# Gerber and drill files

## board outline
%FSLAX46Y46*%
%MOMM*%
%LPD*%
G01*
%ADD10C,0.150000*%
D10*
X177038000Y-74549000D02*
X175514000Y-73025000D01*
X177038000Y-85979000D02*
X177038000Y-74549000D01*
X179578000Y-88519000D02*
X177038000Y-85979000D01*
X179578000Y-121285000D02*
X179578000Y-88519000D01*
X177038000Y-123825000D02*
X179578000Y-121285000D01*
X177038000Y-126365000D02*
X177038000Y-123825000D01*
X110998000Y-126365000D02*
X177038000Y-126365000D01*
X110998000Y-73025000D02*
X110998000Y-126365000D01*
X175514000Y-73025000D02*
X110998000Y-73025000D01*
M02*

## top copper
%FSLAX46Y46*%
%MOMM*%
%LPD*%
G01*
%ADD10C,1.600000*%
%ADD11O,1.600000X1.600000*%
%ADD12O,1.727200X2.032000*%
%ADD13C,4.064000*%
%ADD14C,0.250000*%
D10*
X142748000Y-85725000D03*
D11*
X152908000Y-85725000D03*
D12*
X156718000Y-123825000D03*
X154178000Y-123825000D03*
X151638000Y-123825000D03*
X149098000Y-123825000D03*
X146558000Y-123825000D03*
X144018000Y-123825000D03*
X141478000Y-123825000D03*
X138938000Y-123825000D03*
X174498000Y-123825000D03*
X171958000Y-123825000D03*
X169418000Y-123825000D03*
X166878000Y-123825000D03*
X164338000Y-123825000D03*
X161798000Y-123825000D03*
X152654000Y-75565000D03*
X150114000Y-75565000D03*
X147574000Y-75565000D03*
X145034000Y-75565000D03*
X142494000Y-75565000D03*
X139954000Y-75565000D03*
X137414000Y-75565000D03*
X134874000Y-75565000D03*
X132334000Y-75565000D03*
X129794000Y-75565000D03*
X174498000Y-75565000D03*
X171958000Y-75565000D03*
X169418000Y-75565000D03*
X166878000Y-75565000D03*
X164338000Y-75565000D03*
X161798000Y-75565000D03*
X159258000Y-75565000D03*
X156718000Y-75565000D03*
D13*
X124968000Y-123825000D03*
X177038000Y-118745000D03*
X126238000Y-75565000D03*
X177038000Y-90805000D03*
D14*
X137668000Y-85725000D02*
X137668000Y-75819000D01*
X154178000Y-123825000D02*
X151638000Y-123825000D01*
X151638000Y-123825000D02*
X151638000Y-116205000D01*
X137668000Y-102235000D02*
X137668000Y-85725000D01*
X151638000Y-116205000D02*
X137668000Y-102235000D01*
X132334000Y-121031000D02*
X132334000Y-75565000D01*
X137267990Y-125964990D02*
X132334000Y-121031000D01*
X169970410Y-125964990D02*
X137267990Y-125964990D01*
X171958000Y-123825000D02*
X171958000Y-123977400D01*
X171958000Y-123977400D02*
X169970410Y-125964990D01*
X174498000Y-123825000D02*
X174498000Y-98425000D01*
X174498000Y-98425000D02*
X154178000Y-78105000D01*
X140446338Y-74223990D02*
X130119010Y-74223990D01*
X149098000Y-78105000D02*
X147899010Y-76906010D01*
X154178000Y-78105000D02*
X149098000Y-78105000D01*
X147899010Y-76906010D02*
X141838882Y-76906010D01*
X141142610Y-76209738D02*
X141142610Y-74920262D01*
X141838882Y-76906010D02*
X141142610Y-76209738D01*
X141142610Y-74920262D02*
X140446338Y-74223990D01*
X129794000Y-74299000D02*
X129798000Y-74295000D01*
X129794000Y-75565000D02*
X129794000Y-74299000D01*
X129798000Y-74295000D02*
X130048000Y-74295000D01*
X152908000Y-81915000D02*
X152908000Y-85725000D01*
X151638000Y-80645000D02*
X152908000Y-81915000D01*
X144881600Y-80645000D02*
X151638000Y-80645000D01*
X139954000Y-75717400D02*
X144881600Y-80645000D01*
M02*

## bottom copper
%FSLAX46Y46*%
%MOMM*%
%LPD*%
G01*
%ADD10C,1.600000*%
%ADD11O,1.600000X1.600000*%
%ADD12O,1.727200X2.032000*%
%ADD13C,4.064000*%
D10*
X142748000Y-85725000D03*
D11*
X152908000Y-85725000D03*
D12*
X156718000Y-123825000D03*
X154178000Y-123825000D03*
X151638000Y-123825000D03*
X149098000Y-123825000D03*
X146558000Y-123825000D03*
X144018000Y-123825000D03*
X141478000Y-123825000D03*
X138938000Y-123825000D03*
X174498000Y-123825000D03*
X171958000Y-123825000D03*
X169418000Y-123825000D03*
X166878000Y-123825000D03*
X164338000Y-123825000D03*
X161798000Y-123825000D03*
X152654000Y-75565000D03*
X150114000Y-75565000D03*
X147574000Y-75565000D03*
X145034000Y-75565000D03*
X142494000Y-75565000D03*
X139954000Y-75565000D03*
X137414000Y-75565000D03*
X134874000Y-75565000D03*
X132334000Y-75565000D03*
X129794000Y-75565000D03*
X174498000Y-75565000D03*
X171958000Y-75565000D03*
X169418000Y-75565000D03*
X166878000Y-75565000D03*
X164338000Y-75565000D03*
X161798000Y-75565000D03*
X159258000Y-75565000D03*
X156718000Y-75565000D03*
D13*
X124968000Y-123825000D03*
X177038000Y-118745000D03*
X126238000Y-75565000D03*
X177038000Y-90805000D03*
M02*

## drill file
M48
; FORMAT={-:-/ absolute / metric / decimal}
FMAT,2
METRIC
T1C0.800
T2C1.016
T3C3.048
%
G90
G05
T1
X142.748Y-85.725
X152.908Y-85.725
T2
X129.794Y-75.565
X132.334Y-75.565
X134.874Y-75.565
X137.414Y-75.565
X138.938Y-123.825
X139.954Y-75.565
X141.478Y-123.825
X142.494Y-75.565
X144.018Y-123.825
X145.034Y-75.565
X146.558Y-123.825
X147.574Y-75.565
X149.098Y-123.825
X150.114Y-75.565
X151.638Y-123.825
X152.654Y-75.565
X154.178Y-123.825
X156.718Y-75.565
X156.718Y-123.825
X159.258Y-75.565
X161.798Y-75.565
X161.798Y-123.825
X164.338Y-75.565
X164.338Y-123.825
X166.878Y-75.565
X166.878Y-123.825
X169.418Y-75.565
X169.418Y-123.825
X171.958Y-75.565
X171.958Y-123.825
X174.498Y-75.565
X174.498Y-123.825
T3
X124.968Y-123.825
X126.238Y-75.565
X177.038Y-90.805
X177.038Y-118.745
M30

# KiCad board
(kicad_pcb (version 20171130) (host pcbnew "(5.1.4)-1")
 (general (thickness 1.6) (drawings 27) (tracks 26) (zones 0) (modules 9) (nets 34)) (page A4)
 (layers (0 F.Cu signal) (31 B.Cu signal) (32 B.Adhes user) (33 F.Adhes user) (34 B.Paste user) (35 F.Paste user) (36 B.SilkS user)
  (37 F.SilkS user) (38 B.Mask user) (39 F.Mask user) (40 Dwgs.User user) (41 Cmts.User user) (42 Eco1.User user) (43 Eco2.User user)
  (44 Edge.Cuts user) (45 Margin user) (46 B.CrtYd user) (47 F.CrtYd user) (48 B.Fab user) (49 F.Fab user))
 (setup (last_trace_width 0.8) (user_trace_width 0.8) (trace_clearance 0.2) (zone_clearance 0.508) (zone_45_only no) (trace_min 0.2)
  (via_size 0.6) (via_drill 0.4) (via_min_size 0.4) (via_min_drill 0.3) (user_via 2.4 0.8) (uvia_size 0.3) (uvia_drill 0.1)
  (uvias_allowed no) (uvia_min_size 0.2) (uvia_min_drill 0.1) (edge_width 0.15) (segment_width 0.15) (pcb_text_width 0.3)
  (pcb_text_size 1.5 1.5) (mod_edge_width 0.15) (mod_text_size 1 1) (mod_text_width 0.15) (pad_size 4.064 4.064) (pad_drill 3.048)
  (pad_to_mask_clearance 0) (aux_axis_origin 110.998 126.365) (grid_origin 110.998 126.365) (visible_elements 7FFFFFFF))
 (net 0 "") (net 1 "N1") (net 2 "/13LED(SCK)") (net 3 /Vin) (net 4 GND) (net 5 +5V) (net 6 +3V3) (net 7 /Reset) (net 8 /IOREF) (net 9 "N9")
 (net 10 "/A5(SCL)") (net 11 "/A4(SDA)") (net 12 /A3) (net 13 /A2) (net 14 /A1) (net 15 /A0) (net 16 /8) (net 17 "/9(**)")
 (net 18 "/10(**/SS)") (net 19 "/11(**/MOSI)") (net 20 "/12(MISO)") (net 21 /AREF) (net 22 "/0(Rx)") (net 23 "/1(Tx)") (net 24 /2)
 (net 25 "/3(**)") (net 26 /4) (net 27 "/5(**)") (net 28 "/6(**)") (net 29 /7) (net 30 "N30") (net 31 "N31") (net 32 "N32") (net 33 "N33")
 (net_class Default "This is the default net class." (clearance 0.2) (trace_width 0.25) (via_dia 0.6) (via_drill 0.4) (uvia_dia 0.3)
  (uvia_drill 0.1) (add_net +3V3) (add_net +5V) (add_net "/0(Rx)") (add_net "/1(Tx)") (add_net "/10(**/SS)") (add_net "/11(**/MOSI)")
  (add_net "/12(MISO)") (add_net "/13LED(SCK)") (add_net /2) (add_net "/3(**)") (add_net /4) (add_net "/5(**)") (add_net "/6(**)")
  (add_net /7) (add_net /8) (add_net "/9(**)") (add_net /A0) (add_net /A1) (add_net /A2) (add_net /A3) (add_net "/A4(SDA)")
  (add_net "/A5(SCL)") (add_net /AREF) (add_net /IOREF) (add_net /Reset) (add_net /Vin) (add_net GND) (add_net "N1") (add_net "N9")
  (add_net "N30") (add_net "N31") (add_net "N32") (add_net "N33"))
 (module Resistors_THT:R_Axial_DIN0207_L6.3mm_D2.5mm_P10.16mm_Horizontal (layer F.Cu) (at 142.748 85.725)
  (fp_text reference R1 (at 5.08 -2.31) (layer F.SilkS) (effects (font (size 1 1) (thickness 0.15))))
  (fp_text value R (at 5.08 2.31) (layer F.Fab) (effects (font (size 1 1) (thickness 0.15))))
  (pad 1 thru_hole circle (at 0 0) (size 1.6 1.6) (drill 0.8) (layers *.Cu *.Mask) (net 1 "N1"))
  (pad 2 thru_hole oval (at 10.16 0) (size 1.6 1.6) (drill 0.8) (layers *.Cu *.Mask) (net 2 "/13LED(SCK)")))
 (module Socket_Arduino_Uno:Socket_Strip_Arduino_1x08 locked (layer F.Cu) (at 138.938 123.825)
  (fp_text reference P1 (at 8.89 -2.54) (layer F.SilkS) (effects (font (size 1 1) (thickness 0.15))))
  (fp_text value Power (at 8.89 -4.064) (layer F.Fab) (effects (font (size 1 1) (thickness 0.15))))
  (pad 8 thru_hole oval (at 17.78 0) (size 1.7272 2.032) (drill 1.016) (layers *.Cu *.Mask F.SilkS) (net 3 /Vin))
  (pad 7 thru_hole oval (at 15.24 0) (size 1.7272 2.032) (drill 1.016) (layers *.Cu *.Mask F.SilkS) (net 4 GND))
  (pad 6 thru_hole oval (at 12.7 0) (size 1.7272 2.032) (drill 1.016) (layers *.Cu *.Mask F.SilkS) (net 4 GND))
  (pad 5 thru_hole oval (at 10.16 0) (size 1.7272 2.032) (drill 1.016) (layers *.Cu *.Mask F.SilkS) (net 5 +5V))
  (pad 4 thru_hole oval (at 7.62 0) (size 1.7272 2.032) (drill 1.016) (layers *.Cu *.Mask F.SilkS) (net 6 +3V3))
  (pad 3 thru_hole oval (at 5.08 0) (size 1.7272 2.032) (drill 1.016) (layers *.Cu *.Mask F.SilkS) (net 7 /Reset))
  (pad 2 thru_hole oval (at 2.54 0) (size 1.7272 2.032) (drill 1.016) (layers *.Cu *.Mask F.SilkS) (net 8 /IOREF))
  (pad 1 thru_hole oval (at 0 0) (size 1.7272 2.032) (drill 1.016) (layers *.Cu *.Mask F.SilkS) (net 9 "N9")))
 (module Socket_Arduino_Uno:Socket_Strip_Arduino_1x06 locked (layer F.Cu) (at 161.798 123.825)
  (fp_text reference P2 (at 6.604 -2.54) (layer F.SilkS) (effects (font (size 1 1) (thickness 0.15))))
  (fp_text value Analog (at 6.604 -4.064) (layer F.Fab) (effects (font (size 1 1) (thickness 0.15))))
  (pad 6 thru_hole oval (at 12.7 0) (size 1.7272 2.032) (drill 1.016) (layers *.Cu *.Mask F.SilkS) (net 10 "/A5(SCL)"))
  (pad 5 thru_hole oval (at 10.16 0) (size 1.7272 2.032) (drill 1.016) (layers *.Cu *.Mask F.SilkS) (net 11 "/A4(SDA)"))
  (pad 4 thru_hole oval (at 7.62 0) (size 1.7272 2.032) (drill 1.016) (layers *.Cu *.Mask F.SilkS) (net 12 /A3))
  (pad 3 thru_hole oval (at 5.08 0) (size 1.7272 2.032) (drill 1.016) (layers *.Cu *.Mask F.SilkS) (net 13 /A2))
  (pad 2 thru_hole oval (at 2.54 0) (size 1.7272 2.032) (drill 1.016) (layers *.Cu *.Mask F.SilkS) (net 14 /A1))
  (pad 1 thru_hole oval (at 0 0) (size 1.7272 2.032) (drill 1.016) (layers *.Cu *.Mask F.SilkS) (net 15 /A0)))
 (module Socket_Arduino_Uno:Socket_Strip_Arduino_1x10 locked (layer F.Cu) (at 129.794 75.565)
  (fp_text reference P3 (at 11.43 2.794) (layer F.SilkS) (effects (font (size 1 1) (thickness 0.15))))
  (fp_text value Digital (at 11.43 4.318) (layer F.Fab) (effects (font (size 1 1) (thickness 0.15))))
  (pad 10 thru_hole oval (at 22.86 0) (size 1.7272 2.032) (drill 1.016) (layers *.Cu *.Mask F.SilkS) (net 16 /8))
  (pad 9 thru_hole oval (at 20.32 0) (size 1.7272 2.032) (drill 1.016) (layers *.Cu *.Mask F.SilkS) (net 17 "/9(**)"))
  (pad 8 thru_hole oval (at 17.78 0) (size 1.7272 2.032) (drill 1.016) (layers *.Cu *.Mask F.SilkS) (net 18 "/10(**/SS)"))
  (pad 7 thru_hole oval (at 15.24 0) (size 1.7272 2.032) (drill 1.016) (layers *.Cu *.Mask F.SilkS) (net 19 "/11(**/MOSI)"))
  (pad 6 thru_hole oval (at 12.7 0) (size 1.7272 2.032) (drill 1.016) (layers *.Cu *.Mask F.SilkS) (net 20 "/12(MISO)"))
  (pad 5 thru_hole oval (at 10.16 0) (size 1.7272 2.032) (drill 1.016) (layers *.Cu *.Mask F.SilkS) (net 2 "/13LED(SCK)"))
  (pad 4 thru_hole oval (at 7.62 0) (size 1.7272 2.032) (drill 1.016) (layers *.Cu *.Mask F.SilkS) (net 4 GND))
  (pad 3 thru_hole oval (at 5.08 0) (size 1.7272 2.032) (drill 1.016) (layers *.Cu *.Mask F.SilkS) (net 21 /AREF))
  (pad 2 thru_hole oval (at 2.54 0) (size 1.7272 2.032) (drill 1.016) (layers *.Cu *.Mask F.SilkS) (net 11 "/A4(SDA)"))
  (pad 1 thru_hole oval (at 0 0) (size 1.7272 2.032) (drill 1.016) (layers *.Cu *.Mask F.SilkS) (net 10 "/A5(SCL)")))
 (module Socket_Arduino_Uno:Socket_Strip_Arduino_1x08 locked (layer F.Cu) (at 156.718 75.565)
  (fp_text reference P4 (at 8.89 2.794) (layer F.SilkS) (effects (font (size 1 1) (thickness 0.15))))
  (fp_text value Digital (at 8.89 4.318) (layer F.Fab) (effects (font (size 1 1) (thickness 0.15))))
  (pad 8 thru_hole oval (at 17.78 0) (size 1.7272 2.032) (drill 1.016) (layers *.Cu *.Mask F.SilkS) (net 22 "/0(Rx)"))
  (pad 7 thru_hole oval (at 15.24 0) (size 1.7272 2.032) (drill 1.016) (layers *.Cu *.Mask F.SilkS) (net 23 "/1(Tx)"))
  (pad 6 thru_hole oval (at 12.7 0) (size 1.7272 2.032) (drill 1.016) (layers *.Cu *.Mask F.SilkS) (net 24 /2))
  (pad 5 thru_hole oval (at 10.16 0) (size 1.7272 2.032) (drill 1.016) (layers *.Cu *.Mask F.SilkS) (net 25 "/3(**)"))
  (pad 4 thru_hole oval (at 7.62 0) (size 1.7272 2.032) (drill 1.016) (layers *.Cu *.Mask F.SilkS) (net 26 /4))
  (pad 3 thru_hole oval (at 5.08 0) (size 1.7272 2.032) (drill 1.016) (layers *.Cu *.Mask F.SilkS) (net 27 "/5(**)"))
  (pad 2 thru_hole oval (at 2.54 0) (size 1.7272 2.032) (drill 1.016) (layers *.Cu *.Mask F.SilkS) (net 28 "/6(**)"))
  (pad 1 thru_hole oval (at 0 0) (size 1.7272 2.032) (drill 1.016) (layers *.Cu *.Mask F.SilkS) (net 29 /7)))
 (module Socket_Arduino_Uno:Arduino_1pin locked (layer F.Cu) (at 124.968 123.825)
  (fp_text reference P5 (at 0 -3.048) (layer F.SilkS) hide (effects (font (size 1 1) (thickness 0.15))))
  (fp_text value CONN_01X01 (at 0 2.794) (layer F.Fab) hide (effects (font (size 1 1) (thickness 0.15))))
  (pad 1 thru_hole circle (at 0 0) (size 4.064 4.064) (drill 3.048) (layers *.Cu *.Mask F.SilkS) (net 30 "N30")))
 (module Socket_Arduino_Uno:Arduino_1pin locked (layer F.Cu) (at 177.038 118.745)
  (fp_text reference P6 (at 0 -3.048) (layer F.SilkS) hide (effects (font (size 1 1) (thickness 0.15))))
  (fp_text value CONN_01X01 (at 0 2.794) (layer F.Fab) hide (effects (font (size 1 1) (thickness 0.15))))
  (pad 1 thru_hole circle (at 0 0) (size 4.064 4.064) (drill 3.048) (layers *.Cu *.Mask F.SilkS) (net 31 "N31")))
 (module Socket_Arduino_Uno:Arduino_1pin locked (layer F.Cu) (at 126.238 75.565)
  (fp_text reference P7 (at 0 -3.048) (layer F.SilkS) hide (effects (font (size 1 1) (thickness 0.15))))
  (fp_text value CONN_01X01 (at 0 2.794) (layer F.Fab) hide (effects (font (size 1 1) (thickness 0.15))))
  (pad 1 thru_hole circle (at 0 0) (size 4.064 4.064) (drill 3.048) (layers *.Cu *.Mask F.SilkS) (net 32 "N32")))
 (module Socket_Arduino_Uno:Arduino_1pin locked (layer F.Cu) (at 177.038 90.805)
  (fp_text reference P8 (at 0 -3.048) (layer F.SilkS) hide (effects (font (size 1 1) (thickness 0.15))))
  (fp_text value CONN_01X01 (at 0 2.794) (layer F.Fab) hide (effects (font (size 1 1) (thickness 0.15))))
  (pad 1 thru_hole circle (at 0 0) (size 4.064 4.064) (drill 3.048) (layers *.Cu *.Mask F.SilkS) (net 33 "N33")))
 (gr_line (start 177.038 74.549) (end 175.514 73.025) (angle 90) (layer Edge.Cuts) (width 0.15))
 (gr_line (start 177.038 85.979) (end 177.038 74.549) (angle 90) (layer Edge.Cuts) (width 0.15))
 (gr_line (start 179.578 88.519) (end 177.038 85.979) (angle 90) (layer Edge.Cuts) (width 0.15))
 (gr_line (start 179.578 121.285) (end 179.578 88.519) (angle 90) (layer Edge.Cuts) (width 0.15))
 (gr_line (start 177.038 123.825) (end 179.578 121.285) (angle 90) (layer Edge.Cuts) (width 0.15))
 (gr_line (start 177.038 126.365) (end 177.038 123.825) (angle 90) (layer Edge.Cuts) (width 0.15))
 (gr_line (start 110.998 126.365) (end 177.038 126.365) (angle 90) (layer Edge.Cuts) (width 0.15))
 (gr_line (start 110.998 73.025) (end 110.998 126.365) (angle 90) (layer Edge.Cuts) (width 0.15))
 (gr_line (start 175.514 73.025) (end 110.998 73.025) (angle 90) (layer Edge.Cuts) (width 0.15))
 (segment (start 137.668 85.725) (end 137.668 75.819) (width 0.25) (layer F.Cu) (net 4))
 (segment (start 154.178 123.825) (end 151.638 123.825) (width 0.25) (layer F.Cu) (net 4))
 (segment (start 151.638 123.825) (end 151.638 116.205) (width 0.25) (layer F.Cu) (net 4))
 (segment (start 137.668 102.235) (end 137.668 85.725) (width 0.25) (layer F.Cu) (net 4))
 (segment (start 151.638 116.205) (end 137.668 102.235) (width 0.25) (layer F.Cu) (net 4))
 (segment (start 132.334 121.031) (end 132.334 75.565) (width 0.25) (layer F.Cu) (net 11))
 (segment (start 137.26799 125.96499) (end 132.334 121.031) (width 0.25) (layer F.Cu) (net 11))
 (segment (start 169.97041 125.96499) (end 137.26799 125.96499) (width 0.25) (layer F.Cu) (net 11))
 (segment (start 171.958 123.825) (end 171.958 123.9774) (width 0.25) (layer F.Cu) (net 11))
 (segment (start 171.958 123.9774) (end 169.97041 125.96499) (width 0.25) (layer F.Cu) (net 11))
 (segment (start 174.498 123.825) (end 174.498 98.425) (width 0.25) (layer F.Cu) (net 10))
 (segment (start 174.498 98.425) (end 154.178 78.105) (width 0.25) (layer F.Cu) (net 10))
 (segment (start 140.446338 74.22399) (end 130.11901 74.22399) (width 0.25) (layer F.Cu) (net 10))
 (segment (start 149.098 78.105) (end 147.89901 76.90601) (width 0.25) (layer F.Cu) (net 10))
 (segment (start 154.178 78.105) (end 149.098 78.105) (width 0.25) (layer F.Cu) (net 10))
 (segment (start 147.89901 76.90601) (end 141.838882 76.90601) (width 0.25) (layer F.Cu) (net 10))
 (segment (start 141.14261 76.209738) (end 141.14261 74.920262) (width 0.25) (layer F.Cu) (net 10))
 (segment (start 141.838882 76.90601) (end 141.14261 76.209738) (width 0.25) (layer F.Cu) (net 10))
 (segment (start 141.14261 74.920262) (end 140.446338 74.22399) (width 0.25) (layer F.Cu) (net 10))
 (segment (start 129.794 74.299) (end 129.798 74.295) (width 0.25) (layer F.Cu) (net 10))
 (segment (start 129.794 75.565) (end 129.794 74.299) (width 0.25) (layer F.Cu) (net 10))
 (segment (start 129.798 74.295) (end 130.048 74.295) (width 0.25) (layer F.Cu) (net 10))
 (segment (start 152.908 81.915) (end 152.908 85.725) (width 0.25) (layer F.Cu) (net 2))
 (segment (start 151.638 80.645) (end 152.908 81.915) (width 0.25) (layer F.Cu) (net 2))
 (segment (start 144.8816 80.645) (end 151.638 80.645) (width 0.25) (layer F.Cu) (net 2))
 (segment (start 139.954 75.7174) (end 144.8816 80.645) (width 0.25) (layer F.Cu) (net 2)))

